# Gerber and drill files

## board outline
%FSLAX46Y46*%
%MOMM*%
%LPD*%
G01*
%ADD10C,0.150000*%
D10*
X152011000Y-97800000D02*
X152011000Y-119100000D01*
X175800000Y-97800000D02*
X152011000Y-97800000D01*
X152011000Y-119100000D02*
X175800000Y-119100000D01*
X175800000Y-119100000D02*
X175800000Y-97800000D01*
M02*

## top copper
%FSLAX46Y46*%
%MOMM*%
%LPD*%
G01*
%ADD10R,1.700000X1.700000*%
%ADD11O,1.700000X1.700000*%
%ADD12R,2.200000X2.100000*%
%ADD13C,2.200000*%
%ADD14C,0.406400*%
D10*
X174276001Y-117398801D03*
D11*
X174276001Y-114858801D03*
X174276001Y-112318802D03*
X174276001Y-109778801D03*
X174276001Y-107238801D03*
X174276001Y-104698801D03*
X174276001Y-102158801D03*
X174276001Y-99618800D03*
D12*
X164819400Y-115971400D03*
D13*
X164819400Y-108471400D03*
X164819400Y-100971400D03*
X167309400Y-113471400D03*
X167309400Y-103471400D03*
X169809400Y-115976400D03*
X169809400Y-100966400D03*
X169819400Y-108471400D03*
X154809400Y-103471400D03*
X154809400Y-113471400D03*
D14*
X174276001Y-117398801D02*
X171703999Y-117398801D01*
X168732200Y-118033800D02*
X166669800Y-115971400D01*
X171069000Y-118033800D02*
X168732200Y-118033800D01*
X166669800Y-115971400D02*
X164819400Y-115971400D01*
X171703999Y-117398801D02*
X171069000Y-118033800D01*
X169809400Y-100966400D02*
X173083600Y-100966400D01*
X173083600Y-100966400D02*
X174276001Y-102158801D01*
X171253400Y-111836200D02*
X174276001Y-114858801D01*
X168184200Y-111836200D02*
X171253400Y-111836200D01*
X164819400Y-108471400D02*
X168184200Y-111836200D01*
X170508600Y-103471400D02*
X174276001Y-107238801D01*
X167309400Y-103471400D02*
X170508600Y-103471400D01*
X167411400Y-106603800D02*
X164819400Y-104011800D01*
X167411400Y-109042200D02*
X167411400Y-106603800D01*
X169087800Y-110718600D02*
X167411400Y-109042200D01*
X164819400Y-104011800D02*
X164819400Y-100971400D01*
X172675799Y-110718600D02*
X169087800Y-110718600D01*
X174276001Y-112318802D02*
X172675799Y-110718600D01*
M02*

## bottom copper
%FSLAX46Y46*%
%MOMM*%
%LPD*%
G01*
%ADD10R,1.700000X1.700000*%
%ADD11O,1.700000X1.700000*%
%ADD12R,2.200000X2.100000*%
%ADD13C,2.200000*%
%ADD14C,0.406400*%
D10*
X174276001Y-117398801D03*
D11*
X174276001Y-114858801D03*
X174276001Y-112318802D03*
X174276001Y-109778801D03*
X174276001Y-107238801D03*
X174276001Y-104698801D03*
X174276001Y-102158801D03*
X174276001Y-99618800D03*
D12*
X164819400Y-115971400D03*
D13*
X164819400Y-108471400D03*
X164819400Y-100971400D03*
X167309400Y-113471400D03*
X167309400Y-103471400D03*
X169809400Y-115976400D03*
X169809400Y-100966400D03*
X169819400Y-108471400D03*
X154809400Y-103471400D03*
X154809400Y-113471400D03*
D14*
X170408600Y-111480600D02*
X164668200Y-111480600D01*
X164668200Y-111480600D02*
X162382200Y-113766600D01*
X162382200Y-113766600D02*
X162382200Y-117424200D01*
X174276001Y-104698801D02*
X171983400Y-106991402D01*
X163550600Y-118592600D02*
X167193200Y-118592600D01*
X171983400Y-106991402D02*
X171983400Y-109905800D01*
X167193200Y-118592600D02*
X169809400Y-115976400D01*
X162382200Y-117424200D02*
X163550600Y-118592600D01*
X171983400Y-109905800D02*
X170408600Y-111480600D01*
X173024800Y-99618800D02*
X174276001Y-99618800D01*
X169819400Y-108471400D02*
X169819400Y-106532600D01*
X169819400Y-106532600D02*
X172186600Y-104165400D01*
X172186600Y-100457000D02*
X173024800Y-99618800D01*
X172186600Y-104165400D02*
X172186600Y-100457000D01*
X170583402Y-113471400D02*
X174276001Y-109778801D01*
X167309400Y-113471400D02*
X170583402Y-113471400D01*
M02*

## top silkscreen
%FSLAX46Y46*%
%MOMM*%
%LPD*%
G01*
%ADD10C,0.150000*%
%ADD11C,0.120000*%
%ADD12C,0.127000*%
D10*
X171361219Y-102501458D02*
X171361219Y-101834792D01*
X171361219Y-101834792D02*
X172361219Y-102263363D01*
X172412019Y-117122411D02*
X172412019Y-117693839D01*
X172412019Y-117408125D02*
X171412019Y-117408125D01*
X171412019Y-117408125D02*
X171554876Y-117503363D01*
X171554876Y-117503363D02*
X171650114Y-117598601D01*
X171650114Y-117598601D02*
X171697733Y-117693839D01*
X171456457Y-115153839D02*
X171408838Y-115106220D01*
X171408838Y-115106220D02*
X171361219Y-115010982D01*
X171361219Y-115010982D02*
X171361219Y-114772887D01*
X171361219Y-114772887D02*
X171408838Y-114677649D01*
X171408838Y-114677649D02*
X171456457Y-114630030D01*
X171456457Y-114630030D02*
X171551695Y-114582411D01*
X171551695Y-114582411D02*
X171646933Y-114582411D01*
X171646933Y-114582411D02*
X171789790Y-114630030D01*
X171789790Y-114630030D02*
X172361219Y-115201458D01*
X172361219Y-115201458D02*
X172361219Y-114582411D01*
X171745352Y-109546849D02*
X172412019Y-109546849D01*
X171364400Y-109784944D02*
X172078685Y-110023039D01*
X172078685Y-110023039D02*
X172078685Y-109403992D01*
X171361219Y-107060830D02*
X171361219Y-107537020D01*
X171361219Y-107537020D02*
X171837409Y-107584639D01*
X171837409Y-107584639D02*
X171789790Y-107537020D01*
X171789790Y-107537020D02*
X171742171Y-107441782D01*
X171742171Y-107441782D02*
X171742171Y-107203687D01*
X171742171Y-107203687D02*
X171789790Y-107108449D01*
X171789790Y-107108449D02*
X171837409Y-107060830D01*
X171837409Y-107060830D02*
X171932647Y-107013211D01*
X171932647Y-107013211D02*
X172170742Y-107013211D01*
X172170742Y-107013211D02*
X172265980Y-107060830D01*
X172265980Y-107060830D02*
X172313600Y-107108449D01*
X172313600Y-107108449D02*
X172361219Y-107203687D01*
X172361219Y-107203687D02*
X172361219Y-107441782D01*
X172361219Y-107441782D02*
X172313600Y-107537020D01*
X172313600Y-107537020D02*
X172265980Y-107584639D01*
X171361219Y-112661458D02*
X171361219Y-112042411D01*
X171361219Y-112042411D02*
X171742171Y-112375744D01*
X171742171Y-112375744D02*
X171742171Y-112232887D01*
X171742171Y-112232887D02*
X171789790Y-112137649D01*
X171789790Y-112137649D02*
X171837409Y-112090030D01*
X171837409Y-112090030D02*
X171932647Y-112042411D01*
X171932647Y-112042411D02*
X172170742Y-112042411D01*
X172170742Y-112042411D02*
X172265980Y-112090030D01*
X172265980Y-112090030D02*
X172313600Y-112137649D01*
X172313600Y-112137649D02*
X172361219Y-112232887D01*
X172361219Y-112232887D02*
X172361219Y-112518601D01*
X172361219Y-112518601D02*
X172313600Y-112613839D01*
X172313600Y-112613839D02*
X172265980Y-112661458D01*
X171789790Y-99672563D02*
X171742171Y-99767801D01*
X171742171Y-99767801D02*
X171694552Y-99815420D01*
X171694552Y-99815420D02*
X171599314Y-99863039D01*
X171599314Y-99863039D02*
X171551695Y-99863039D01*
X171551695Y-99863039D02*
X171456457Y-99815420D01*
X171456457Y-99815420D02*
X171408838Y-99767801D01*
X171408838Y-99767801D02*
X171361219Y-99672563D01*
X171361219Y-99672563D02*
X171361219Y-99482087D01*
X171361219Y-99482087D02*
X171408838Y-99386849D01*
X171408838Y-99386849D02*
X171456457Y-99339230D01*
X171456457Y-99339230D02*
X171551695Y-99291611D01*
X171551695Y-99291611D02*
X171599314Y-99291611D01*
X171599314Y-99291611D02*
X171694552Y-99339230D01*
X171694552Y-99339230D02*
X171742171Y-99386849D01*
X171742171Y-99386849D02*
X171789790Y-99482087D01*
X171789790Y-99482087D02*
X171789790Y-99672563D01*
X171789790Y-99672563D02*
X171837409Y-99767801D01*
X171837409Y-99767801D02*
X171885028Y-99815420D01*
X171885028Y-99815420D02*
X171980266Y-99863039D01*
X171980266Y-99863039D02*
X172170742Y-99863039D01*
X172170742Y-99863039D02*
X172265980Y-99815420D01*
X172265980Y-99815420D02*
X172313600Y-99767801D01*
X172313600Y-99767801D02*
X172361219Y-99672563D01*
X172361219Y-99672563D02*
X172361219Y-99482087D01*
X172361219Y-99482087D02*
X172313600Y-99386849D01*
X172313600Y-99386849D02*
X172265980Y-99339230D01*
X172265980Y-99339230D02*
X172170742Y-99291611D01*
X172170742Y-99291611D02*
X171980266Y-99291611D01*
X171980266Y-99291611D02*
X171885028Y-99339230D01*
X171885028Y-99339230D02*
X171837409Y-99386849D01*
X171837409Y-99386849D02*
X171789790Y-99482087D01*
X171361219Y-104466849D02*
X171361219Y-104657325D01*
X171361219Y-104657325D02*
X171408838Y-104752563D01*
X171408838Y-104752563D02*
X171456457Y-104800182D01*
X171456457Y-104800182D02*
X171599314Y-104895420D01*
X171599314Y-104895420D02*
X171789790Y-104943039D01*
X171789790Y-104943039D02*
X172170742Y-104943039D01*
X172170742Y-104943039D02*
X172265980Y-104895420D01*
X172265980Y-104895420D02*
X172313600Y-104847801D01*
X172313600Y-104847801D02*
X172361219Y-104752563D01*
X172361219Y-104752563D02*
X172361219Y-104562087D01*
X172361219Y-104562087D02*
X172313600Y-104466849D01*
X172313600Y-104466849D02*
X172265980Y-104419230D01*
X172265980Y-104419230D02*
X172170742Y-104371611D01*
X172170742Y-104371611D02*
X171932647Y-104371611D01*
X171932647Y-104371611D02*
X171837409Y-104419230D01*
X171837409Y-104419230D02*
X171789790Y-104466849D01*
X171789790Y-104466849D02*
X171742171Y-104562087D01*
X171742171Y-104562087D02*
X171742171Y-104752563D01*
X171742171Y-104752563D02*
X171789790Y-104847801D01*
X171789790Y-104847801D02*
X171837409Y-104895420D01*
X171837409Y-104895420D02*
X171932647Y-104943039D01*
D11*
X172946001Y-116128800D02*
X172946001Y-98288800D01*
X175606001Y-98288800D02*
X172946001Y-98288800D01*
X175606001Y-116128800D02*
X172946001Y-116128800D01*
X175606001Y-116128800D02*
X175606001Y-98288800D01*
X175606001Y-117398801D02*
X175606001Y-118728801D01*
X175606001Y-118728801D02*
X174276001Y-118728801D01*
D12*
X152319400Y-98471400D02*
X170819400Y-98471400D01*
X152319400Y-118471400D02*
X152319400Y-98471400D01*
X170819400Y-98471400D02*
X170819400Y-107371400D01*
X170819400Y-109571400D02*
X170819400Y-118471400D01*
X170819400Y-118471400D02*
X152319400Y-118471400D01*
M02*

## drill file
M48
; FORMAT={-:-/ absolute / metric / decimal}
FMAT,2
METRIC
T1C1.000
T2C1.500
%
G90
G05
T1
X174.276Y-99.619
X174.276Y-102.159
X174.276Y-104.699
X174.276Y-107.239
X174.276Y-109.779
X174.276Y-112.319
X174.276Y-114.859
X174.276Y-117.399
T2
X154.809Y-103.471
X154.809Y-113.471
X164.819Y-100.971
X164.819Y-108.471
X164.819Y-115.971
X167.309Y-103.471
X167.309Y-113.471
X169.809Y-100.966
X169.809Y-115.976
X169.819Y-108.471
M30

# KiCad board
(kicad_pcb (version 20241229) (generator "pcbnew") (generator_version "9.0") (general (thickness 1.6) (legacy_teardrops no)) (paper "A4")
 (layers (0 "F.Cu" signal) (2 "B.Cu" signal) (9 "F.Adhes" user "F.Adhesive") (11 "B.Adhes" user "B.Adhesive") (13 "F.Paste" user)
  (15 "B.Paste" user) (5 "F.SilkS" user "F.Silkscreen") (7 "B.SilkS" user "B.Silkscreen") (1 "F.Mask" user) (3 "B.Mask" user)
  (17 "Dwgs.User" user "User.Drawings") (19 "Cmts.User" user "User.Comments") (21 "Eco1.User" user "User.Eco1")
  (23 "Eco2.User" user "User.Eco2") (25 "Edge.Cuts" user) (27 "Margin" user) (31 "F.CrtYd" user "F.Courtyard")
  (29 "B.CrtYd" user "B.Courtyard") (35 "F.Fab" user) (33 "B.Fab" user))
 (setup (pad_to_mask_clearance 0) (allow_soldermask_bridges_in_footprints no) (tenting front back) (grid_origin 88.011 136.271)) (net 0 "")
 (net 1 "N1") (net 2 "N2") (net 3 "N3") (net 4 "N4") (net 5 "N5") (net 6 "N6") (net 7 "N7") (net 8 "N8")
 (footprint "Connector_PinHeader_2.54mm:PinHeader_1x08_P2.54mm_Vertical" (layer "F.Cu") (at 174.276001 117.398801 180)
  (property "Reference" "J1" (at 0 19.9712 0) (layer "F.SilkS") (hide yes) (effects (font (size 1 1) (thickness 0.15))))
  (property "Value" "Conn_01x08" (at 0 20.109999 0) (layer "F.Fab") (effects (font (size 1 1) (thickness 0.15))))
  (fp_line (start 1.33 1.270001) (end 1.33 19.110001) (stroke (width 0.12) (type solid)) (layer "F.SilkS"))
  (fp_line (start -1.33 19.110001) (end 1.33 19.110001) (stroke (width 0.12) (type solid)) (layer "F.SilkS"))
  (fp_line (start -1.33 1.270001) (end 1.33 1.270001) (stroke (width 0.12) (type solid)) (layer "F.SilkS"))
  (fp_line (start -1.33 1.270001) (end -1.33 19.110001) (stroke (width 0.12) (type solid)) (layer "F.SilkS"))
  (fp_line (start -1.33 0) (end -1.33 -1.33) (stroke (width 0.12) (type solid)) (layer "F.SilkS"))
  (fp_line (start -1.33 -1.33) (end 0 -1.33) (stroke (width 0.12) (type solid)) (layer "F.SilkS"))
  (pad "1" thru_hole rect (at 0 0 180) (size 1.7 1.7) (drill 1) (layers "*.Cu" "*.Mask") (remove_unused_layers no) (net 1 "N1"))
  (pad "2" thru_hole oval (at 0 2.54 180) (size 1.7 1.7) (drill 1) (layers "*.Cu" "*.Mask") (remove_unused_layers no) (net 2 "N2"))
  (pad "3" thru_hole oval (at 0 5.079999 180) (size 1.7 1.7) (drill 1) (layers "*.Cu" "*.Mask") (remove_unused_layers no) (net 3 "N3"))
  (pad "4" thru_hole oval (at 0 7.62 180) (size 1.7 1.7) (drill 1) (layers "*.Cu" "*.Mask") (remove_unused_layers no) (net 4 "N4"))
  (pad "5" thru_hole oval (at 0 10.16 180) (size 1.7 1.7) (drill 1) (layers "*.Cu" "*.Mask") (remove_unused_layers no) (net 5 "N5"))
  (pad "6" thru_hole oval (at 0 12.7 180) (size 1.7 1.7) (drill 1) (layers "*.Cu" "*.Mask") (remove_unused_layers no) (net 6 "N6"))
  (pad "7" thru_hole oval (at 0 15.24 180) (size 1.7 1.7) (drill 1) (layers "*.Cu" "*.Mask") (remove_unused_layers no) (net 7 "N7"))
  (pad "8" thru_hole oval (at 0 17.780001 180) (size 1.7 1.7) (drill 1) (layers "*.Cu" "*.Mask") (remove_unused_layers no) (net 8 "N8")))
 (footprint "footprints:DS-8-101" (layer "F.Cu") (at 159.8094 108.4714)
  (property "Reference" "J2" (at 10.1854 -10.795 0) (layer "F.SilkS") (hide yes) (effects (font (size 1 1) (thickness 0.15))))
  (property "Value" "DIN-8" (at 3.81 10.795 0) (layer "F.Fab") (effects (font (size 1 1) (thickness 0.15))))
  (fp_line (start -7.49 -10) (end 11.01 -10) (stroke (width 0.127) (type solid)) (layer "F.SilkS"))
  (fp_line (start -7.49 10) (end -7.49 -10) (stroke (width 0.127) (type solid)) (layer "F.SilkS"))
  (fp_line (start 11.01 -10) (end 11.01 -1.1) (stroke (width 0.127) (type solid)) (layer "F.SilkS"))
  (fp_line (start 11.01 1.1) (end 11.01 10) (stroke (width 0.127) (type solid)) (layer "F.SilkS"))
  (fp_line (start 11.01 10) (end -7.49 10) (stroke (width 0.127) (type solid)) (layer "F.SilkS"))
  (pad "1" thru_hole rect (at 5.01 7.5) (size 2.2 2.1) (drill 1.5) (layers "*.Cu" "*.Mask") (remove_unused_layers no) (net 1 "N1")
   (solder_mask_margin 0.102))
  (pad "2" thru_hole circle (at 5.01 0) (size 2.2 2.2) (drill 1.5) (layers "*.Cu" "*.Mask") (remove_unused_layers no) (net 2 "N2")
   (solder_mask_margin 0.102))
  (pad "3" thru_hole circle (at 5.01 -7.5) (size 2.2 2.2) (drill 1.5) (layers "*.Cu" "*.Mask") (remove_unused_layers no) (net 3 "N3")
   (solder_mask_margin 0.102))
  (pad "4" thru_hole circle (at 7.5 5) (size 2.2 2.2) (drill 1.5) (layers "*.Cu" "*.Mask") (remove_unused_layers no) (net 4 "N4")
   (solder_mask_margin 0.102))
  (pad "5" thru_hole circle (at 7.5 -5) (size 2.2 2.2) (drill 1.5) (layers "*.Cu" "*.Mask") (remove_unused_layers no) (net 5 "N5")
   (solder_mask_margin 0.102))
  (pad "6" thru_hole circle (at 10 7.505) (size 2.2 2.2) (drill 1.5) (layers "*.Cu" "*.Mask") (remove_unused_layers no) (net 6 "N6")
   (solder_mask_margin 0.102))
  (pad "7" thru_hole circle (at 10 -7.505) (size 2.2 2.2) (drill 1.5) (layers "*.Cu" "*.Mask") (remove_unused_layers no) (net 7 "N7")
   (solder_mask_margin 0.102))
  (pad "8" thru_hole circle (at 10.01 0) (size 2.2 2.2) (drill 1.5) (layers "*.Cu" "*.Mask") (remove_unused_layers no) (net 8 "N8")
   (solder_mask_margin 0.102))
  (pad "G1" thru_hole circle (at -5 -5) (size 2.2 2.2) (drill 1.5) (layers "*.Cu" "*.Mask") (remove_unused_layers no)
   (solder_mask_margin 0.102))
  (pad "G2" thru_hole circle (at -5 5) (size 2.2 2.2) (drill 1.5) (layers "*.Cu" "*.Mask") (remove_unused_layers no)
   (solder_mask_margin 0.102)))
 (gr_line (start 152.011 97.8) (end 152.011 119.1) (stroke (width 0.15) (type solid)) (layer "Edge.Cuts"))
 (gr_line (start 175.8 97.8) (end 152.011 97.8) (stroke (width 0.15) (type solid)) (layer "Edge.Cuts"))
 (gr_line (start 152.011 119.1) (end 175.8 119.1) (stroke (width 0.15) (type solid)) (layer "Edge.Cuts"))
 (gr_line (start 175.8 119.1) (end 175.8 97.8) (stroke (width 0.15) (type solid)) (layer "Edge.Cuts"))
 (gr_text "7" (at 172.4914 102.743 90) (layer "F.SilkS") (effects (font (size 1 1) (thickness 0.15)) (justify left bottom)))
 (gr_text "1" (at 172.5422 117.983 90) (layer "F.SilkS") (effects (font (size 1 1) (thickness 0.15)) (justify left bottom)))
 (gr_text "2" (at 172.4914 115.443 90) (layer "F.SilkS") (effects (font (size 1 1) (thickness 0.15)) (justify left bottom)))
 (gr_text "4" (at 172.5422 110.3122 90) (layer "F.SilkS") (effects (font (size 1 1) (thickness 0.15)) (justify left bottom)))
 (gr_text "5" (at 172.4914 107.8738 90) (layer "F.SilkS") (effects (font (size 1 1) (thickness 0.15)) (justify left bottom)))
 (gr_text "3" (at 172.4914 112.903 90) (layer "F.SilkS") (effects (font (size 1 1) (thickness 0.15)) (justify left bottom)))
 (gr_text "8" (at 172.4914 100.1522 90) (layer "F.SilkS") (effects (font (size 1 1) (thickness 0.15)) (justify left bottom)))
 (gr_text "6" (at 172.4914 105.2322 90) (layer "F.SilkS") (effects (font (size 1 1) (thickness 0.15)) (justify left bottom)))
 (segment (start 170.4086 111.4806) (end 164.6682 111.4806) (width 0.4064) (layer "B.Cu") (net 6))
 (segment (start 164.6682 111.4806) (end 162.3822 113.7666) (width 0.4064) (layer "B.Cu") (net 6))
 (segment (start 162.3822 113.7666) (end 162.3822 117.4242) (width 0.4064) (layer "B.Cu") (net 6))
 (segment (start 174.276001 104.698801) (end 171.9834 106.991402) (width 0.4064) (layer "B.Cu") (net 6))
 (segment (start 163.5506 118.5926) (end 167.1932 118.5926) (width 0.4064) (layer "B.Cu") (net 6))
 (segment (start 171.9834 106.991402) (end 171.9834 109.9058) (width 0.4064) (layer "B.Cu") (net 6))
 (segment (start 167.1932 118.5926) (end 169.8094 115.9764) (width 0.4064) (layer "B.Cu") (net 6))
 (segment (start 162.3822 117.4242) (end 163.5506 118.5926) (width 0.4064) (layer "B.Cu") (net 6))
 (segment (start 171.9834 109.9058) (end 170.4086 111.4806) (width 0.4064) (layer "B.Cu") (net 6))
 (segment (start 174.276001 117.398801) (end 171.703999 117.398801) (width 0.4064) (layer "F.Cu") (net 1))
 (segment (start 168.7322 118.0338) (end 166.6698 115.9714) (width 0.4064) (layer "F.Cu") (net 1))
 (segment (start 171.069 118.0338) (end 168.7322 118.0338) (width 0.4064) (layer "F.Cu") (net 1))
 (segment (start 166.6698 115.9714) (end 164.8194 115.9714) (width 0.4064) (layer "F.Cu") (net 1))
 (segment (start 171.703999 117.398801) (end 171.069 118.0338) (width 0.4064) (layer "F.Cu") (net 1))
 (segment (start 169.8094 100.9664) (end 173.0836 100.9664) (width 0.4064) (layer "F.Cu") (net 7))
 (segment (start 173.0836 100.9664) (end 174.276001 102.158801) (width 0.4064) (layer "F.Cu") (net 7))
 (segment (start 173.0248 99.6188) (end 174.276001 99.6188) (width 0.4064) (layer "B.Cu") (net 8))
 (segment (start 169.8194 108.4714) (end 169.8194 106.5326) (width 0.4064) (layer "B.Cu") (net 8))
 (segment (start 169.8194 106.5326) (end 172.1866 104.1654) (width 0.4064) (layer "B.Cu") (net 8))
 (segment (start 172.1866 100.457) (end 173.0248 99.6188) (width 0.4064) (layer "B.Cu") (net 8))
 (segment (start 172.1866 104.1654) (end 172.1866 100.457) (width 0.4064) (layer "B.Cu") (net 8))
 (segment (start 170.583402 113.4714) (end 174.276001 109.778801) (width 0.4064) (layer "B.Cu") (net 4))
 (segment (start 167.3094 113.4714) (end 170.583402 113.4714) (width 0.4064) (layer "B.Cu") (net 4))
 (segment (start 171.2534 111.8362) (end 174.276001 114.858801) (width 0.4064) (layer "F.Cu") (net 2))
 (segment (start 168.1842 111.8362) (end 171.2534 111.8362) (width 0.4064) (layer "F.Cu") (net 2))
 (segment (start 164.8194 108.4714) (end 168.1842 111.8362) (width 0.4064) (layer "F.Cu") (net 2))
 (segment (start 170.5086 103.4714) (end 174.276001 107.238801) (width 0.4064) (layer "F.Cu") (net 5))
 (segment (start 167.3094 103.4714) (end 170.5086 103.4714) (width 0.4064) (layer "F.Cu") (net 5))
 (segment (start 167.4114 106.6038) (end 164.8194 104.0118) (width 0.4064) (layer "F.Cu") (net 3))
 (segment (start 167.4114 109.0422) (end 167.4114 106.6038) (width 0.4064) (layer "F.Cu") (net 3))
 (segment (start 169.0878 110.7186) (end 167.4114 109.0422) (width 0.4064) (layer "F.Cu") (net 3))
 (segment (start 164.8194 104.0118) (end 164.8194 100.9714) (width 0.4064) (layer "F.Cu") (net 3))
 (segment (start 172.675799 110.7186) (end 169.0878 110.7186) (width 0.4064) (layer "F.Cu") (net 3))
 (segment (start 174.276001 112.318802) (end 172.675799 110.7186) (width 0.4064) (layer "F.Cu") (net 3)))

